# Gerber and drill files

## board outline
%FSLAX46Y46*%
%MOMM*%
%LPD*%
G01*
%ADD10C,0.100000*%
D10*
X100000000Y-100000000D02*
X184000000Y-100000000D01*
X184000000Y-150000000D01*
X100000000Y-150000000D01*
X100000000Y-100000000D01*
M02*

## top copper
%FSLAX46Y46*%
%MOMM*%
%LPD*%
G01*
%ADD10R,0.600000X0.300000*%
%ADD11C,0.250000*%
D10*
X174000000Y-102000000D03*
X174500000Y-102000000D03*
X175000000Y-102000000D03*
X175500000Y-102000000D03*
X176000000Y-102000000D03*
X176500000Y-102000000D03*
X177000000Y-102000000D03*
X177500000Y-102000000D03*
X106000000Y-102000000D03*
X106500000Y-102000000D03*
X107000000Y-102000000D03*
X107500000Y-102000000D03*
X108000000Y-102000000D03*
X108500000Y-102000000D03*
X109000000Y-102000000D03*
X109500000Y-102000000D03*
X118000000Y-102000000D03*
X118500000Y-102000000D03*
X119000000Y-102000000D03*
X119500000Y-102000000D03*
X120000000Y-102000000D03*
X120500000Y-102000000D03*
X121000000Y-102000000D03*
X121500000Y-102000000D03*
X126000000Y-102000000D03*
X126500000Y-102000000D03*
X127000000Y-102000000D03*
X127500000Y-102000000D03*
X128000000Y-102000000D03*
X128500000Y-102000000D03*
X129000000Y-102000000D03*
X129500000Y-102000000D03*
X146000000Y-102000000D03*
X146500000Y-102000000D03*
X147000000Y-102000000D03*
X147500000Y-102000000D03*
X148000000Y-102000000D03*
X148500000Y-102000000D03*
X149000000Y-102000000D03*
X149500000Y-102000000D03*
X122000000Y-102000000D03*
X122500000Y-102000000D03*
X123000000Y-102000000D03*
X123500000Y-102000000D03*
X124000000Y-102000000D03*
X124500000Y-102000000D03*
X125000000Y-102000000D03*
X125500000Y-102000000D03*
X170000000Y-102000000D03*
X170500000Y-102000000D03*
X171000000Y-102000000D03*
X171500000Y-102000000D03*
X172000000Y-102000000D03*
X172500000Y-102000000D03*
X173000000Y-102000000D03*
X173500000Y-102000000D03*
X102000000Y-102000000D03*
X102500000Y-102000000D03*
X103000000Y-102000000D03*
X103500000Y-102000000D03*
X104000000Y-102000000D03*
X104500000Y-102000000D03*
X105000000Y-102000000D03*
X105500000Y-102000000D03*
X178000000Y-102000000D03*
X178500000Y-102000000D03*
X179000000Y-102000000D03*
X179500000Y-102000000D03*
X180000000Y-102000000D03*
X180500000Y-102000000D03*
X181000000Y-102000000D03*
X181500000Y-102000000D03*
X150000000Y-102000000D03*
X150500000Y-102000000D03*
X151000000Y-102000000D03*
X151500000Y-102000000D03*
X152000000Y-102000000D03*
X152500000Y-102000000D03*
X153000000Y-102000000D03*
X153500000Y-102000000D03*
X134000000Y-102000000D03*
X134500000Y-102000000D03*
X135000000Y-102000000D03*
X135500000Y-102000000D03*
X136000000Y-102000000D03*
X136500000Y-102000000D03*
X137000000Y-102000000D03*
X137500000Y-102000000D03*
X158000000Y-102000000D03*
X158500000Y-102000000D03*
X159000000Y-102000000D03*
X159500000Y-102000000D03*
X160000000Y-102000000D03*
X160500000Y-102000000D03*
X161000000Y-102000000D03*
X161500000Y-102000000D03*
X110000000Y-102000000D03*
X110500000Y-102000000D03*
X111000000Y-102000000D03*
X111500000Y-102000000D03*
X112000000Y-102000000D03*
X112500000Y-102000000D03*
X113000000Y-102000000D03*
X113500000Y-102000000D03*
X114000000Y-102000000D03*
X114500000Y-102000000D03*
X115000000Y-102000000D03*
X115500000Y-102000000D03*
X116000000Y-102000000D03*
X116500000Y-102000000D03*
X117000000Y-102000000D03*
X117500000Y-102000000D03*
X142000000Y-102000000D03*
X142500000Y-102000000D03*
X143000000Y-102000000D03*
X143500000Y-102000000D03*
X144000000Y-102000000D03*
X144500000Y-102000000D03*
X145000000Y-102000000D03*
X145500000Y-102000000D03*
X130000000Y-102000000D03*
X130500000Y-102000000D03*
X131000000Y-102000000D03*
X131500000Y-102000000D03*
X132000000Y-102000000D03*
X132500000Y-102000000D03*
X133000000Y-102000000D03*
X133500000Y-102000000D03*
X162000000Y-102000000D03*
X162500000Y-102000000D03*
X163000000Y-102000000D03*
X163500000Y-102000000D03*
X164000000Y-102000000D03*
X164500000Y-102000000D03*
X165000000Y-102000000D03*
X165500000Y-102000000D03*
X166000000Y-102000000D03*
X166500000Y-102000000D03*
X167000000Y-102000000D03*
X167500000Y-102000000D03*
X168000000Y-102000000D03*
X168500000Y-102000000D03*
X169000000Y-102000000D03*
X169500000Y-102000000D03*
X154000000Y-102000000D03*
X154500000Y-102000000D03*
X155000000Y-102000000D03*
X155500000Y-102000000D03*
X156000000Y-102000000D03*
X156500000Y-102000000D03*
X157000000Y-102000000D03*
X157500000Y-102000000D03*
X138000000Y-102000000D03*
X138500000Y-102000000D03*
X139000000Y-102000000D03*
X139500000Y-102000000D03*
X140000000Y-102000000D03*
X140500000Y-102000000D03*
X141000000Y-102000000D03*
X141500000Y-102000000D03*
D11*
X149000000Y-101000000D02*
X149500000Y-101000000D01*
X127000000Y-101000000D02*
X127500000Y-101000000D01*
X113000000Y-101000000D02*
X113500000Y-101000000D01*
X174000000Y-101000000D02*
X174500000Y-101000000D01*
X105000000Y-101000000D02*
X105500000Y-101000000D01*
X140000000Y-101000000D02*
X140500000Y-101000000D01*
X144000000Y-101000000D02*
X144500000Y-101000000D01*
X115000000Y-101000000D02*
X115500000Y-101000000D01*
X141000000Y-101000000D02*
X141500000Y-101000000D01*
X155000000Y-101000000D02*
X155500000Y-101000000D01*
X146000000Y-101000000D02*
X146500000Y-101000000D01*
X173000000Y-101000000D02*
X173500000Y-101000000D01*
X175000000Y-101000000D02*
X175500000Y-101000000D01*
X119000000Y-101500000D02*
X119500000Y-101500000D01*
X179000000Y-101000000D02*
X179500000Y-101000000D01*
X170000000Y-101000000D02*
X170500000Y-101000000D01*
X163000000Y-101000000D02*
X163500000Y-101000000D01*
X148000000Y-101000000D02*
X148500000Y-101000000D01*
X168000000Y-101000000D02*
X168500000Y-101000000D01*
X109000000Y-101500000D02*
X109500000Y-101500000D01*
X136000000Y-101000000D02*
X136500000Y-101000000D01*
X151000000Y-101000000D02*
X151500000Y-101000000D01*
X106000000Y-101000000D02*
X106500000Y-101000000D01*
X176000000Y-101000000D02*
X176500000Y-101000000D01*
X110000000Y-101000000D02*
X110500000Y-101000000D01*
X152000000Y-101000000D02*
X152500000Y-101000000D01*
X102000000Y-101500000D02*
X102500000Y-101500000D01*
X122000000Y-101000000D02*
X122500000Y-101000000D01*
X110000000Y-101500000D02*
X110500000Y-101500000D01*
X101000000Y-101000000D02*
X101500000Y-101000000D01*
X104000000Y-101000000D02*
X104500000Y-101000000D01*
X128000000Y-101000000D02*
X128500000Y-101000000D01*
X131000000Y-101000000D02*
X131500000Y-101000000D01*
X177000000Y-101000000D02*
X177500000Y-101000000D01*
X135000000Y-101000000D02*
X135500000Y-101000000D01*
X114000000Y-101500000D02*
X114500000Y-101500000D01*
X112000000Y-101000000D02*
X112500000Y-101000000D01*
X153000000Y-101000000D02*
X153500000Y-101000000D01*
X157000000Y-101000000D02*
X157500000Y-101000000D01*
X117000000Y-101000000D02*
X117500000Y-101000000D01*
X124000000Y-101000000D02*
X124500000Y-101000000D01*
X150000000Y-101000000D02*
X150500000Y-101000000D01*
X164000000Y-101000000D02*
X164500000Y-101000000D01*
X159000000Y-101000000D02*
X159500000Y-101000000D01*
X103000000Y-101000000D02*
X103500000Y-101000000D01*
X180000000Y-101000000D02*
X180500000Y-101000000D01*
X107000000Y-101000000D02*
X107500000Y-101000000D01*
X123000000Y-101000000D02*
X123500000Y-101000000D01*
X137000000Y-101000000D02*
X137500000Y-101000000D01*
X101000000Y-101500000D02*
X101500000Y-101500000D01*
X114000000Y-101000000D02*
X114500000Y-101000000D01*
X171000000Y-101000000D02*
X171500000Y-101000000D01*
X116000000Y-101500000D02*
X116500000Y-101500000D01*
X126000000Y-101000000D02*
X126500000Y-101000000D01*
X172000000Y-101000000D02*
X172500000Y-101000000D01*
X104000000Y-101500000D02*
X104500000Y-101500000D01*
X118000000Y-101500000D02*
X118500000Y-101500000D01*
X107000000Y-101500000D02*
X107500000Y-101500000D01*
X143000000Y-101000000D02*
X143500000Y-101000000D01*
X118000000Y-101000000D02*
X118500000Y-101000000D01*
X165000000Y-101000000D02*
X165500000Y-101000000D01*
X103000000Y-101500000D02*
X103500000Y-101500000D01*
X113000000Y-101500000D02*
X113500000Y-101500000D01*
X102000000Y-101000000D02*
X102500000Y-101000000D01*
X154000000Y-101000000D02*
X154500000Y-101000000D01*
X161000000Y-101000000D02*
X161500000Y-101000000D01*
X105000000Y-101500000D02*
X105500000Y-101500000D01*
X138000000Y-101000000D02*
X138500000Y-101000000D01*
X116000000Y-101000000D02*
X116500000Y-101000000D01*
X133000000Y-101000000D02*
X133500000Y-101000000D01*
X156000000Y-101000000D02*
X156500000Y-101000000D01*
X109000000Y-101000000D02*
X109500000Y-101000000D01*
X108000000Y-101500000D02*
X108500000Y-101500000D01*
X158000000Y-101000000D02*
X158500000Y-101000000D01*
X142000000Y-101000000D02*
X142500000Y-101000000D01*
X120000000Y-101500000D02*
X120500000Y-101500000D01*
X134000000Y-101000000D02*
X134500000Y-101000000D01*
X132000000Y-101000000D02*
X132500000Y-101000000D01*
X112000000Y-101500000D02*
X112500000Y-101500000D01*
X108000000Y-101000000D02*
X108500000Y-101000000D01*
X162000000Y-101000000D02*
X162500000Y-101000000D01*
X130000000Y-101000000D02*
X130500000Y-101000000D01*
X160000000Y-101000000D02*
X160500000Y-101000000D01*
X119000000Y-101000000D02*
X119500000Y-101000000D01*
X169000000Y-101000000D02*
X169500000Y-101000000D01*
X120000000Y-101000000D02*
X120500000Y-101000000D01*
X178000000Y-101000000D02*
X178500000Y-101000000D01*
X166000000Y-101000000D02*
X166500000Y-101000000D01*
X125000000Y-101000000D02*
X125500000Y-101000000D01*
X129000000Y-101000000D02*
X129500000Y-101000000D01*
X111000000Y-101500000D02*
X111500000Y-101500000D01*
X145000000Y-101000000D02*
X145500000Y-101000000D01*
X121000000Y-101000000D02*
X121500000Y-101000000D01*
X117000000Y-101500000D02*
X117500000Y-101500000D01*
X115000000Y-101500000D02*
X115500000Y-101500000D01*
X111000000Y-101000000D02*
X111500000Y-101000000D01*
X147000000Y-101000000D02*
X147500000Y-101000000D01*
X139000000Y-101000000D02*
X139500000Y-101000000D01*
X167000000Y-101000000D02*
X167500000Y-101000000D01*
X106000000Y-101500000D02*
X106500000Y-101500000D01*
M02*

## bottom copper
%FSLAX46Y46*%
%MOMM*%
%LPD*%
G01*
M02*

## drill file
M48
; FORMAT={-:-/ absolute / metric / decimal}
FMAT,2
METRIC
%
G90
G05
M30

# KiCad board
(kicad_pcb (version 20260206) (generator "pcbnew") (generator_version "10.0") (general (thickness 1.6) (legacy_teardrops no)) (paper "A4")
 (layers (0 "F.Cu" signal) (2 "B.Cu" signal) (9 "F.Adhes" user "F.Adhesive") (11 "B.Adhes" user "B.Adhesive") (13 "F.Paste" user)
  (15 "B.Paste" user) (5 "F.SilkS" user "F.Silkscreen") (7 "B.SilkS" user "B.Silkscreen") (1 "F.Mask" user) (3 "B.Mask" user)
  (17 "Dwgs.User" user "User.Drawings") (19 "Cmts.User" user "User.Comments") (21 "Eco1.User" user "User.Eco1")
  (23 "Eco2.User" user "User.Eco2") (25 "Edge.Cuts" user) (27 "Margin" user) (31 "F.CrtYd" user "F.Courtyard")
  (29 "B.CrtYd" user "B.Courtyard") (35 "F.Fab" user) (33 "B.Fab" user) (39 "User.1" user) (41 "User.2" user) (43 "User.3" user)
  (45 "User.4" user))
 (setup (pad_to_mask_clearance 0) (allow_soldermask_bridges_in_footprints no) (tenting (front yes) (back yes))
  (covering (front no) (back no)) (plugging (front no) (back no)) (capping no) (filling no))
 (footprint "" (layer "F.Cu") (at 174 102)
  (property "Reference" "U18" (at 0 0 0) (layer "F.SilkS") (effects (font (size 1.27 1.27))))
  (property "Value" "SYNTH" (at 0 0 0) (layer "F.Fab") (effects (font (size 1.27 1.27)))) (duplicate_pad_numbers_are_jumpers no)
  (pad "1" smd rect (at 0 0) (size 0.6 0.3) (layers "F.Cu" "F.Mask" "F.Paste") (thermal_bridge_angle 45))
  (pad "2" smd rect (at 0.5 0) (size 0.6 0.3) (layers "F.Cu" "F.Mask" "F.Paste") (thermal_bridge_angle 45))
  (pad "3" smd rect (at 1 0) (size 0.6 0.3) (layers "F.Cu" "F.Mask" "F.Paste") (thermal_bridge_angle 45))
  (pad "4" smd rect (at 1.5 0) (size 0.6 0.3) (layers "F.Cu" "F.Mask" "F.Paste") (thermal_bridge_angle 45))
  (pad "5" smd rect (at 2 0) (size 0.6 0.3) (layers "F.Cu" "F.Mask" "F.Paste") (thermal_bridge_angle 45))
  (pad "6" smd rect (at 2.5 0) (size 0.6 0.3) (layers "F.Cu" "F.Mask" "F.Paste") (thermal_bridge_angle 45))
  (pad "7" smd rect (at 3 0) (size 0.6 0.3) (layers "F.Cu" "F.Mask" "F.Paste") (thermal_bridge_angle 45))
  (pad "8" smd rect (at 3.5 0) (size 0.6 0.3) (layers "F.Cu" "F.Mask" "F.Paste") (thermal_bridge_angle 45)))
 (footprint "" (layer "F.Cu") (at 106 102)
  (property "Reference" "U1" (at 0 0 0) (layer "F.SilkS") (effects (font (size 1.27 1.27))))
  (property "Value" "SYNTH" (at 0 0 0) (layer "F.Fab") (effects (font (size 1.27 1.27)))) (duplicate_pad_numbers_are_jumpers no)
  (pad "1" smd rect (at 0 0) (size 0.6 0.3) (layers "F.Cu" "F.Mask" "F.Paste") (thermal_bridge_angle 45))
  (pad "2" smd rect (at 0.5 0) (size 0.6 0.3) (layers "F.Cu" "F.Mask" "F.Paste") (thermal_bridge_angle 45))
  (pad "3" smd rect (at 1 0) (size 0.6 0.3) (layers "F.Cu" "F.Mask" "F.Paste") (thermal_bridge_angle 45))
  (pad "4" smd rect (at 1.5 0) (size 0.6 0.3) (layers "F.Cu" "F.Mask" "F.Paste") (thermal_bridge_angle 45))
  (pad "5" smd rect (at 2 0) (size 0.6 0.3) (layers "F.Cu" "F.Mask" "F.Paste") (thermal_bridge_angle 45))
  (pad "6" smd rect (at 2.5 0) (size 0.6 0.3) (layers "F.Cu" "F.Mask" "F.Paste") (thermal_bridge_angle 45))
  (pad "7" smd rect (at 3 0) (size 0.6 0.3) (layers "F.Cu" "F.Mask" "F.Paste") (thermal_bridge_angle 45))
  (pad "8" smd rect (at 3.5 0) (size 0.6 0.3) (layers "F.Cu" "F.Mask" "F.Paste") (thermal_bridge_angle 45)))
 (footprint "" (layer "F.Cu") (at 118 102)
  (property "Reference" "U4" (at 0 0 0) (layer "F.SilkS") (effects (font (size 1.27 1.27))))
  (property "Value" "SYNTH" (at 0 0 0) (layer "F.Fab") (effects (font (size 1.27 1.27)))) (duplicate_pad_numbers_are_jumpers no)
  (pad "1" smd rect (at 0 0) (size 0.6 0.3) (layers "F.Cu" "F.Mask" "F.Paste") (thermal_bridge_angle 45))
  (pad "2" smd rect (at 0.5 0) (size 0.6 0.3) (layers "F.Cu" "F.Mask" "F.Paste") (thermal_bridge_angle 45))
  (pad "3" smd rect (at 1 0) (size 0.6 0.3) (layers "F.Cu" "F.Mask" "F.Paste") (thermal_bridge_angle 45))
  (pad "4" smd rect (at 1.5 0) (size 0.6 0.3) (layers "F.Cu" "F.Mask" "F.Paste") (thermal_bridge_angle 45))
  (pad "5" smd rect (at 2 0) (size 0.6 0.3) (layers "F.Cu" "F.Mask" "F.Paste") (thermal_bridge_angle 45))
  (pad "6" smd rect (at 2.5 0) (size 0.6 0.3) (layers "F.Cu" "F.Mask" "F.Paste") (thermal_bridge_angle 45))
  (pad "7" smd rect (at 3 0) (size 0.6 0.3) (layers "F.Cu" "F.Mask" "F.Paste") (thermal_bridge_angle 45))
  (pad "8" smd rect (at 3.5 0) (size 0.6 0.3) (layers "F.Cu" "F.Mask" "F.Paste") (thermal_bridge_angle 45)))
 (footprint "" (layer "F.Cu") (at 126 102)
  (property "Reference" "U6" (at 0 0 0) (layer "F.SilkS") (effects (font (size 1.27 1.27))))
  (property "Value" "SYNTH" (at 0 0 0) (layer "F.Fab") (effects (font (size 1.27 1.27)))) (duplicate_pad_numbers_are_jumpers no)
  (pad "1" smd rect (at 0 0) (size 0.6 0.3) (layers "F.Cu" "F.Mask" "F.Paste") (thermal_bridge_angle 45))
  (pad "2" smd rect (at 0.5 0) (size 0.6 0.3) (layers "F.Cu" "F.Mask" "F.Paste") (thermal_bridge_angle 45))
  (pad "3" smd rect (at 1 0) (size 0.6 0.3) (layers "F.Cu" "F.Mask" "F.Paste") (thermal_bridge_angle 45))
  (pad "4" smd rect (at 1.5 0) (size 0.6 0.3) (layers "F.Cu" "F.Mask" "F.Paste") (thermal_bridge_angle 45))
  (pad "5" smd rect (at 2 0) (size 0.6 0.3) (layers "F.Cu" "F.Mask" "F.Paste") (thermal_bridge_angle 45))
  (pad "6" smd rect (at 2.5 0) (size 0.6 0.3) (layers "F.Cu" "F.Mask" "F.Paste") (thermal_bridge_angle 45))
  (pad "7" smd rect (at 3 0) (size 0.6 0.3) (layers "F.Cu" "F.Mask" "F.Paste") (thermal_bridge_angle 45))
  (pad "8" smd rect (at 3.5 0) (size 0.6 0.3) (layers "F.Cu" "F.Mask" "F.Paste") (thermal_bridge_angle 45)))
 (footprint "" (layer "F.Cu") (at 146 102)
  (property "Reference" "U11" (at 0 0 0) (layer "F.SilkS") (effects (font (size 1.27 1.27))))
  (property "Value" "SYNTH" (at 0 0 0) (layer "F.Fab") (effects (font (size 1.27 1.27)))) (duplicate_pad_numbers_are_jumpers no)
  (pad "1" smd rect (at 0 0) (size 0.6 0.3) (layers "F.Cu" "F.Mask" "F.Paste") (thermal_bridge_angle 45))
  (pad "2" smd rect (at 0.5 0) (size 0.6 0.3) (layers "F.Cu" "F.Mask" "F.Paste") (thermal_bridge_angle 45))
  (pad "3" smd rect (at 1 0) (size 0.6 0.3) (layers "F.Cu" "F.Mask" "F.Paste") (thermal_bridge_angle 45))
  (pad "4" smd rect (at 1.5 0) (size 0.6 0.3) (layers "F.Cu" "F.Mask" "F.Paste") (thermal_bridge_angle 45))
  (pad "5" smd rect (at 2 0) (size 0.6 0.3) (layers "F.Cu" "F.Mask" "F.Paste") (thermal_bridge_angle 45))
  (pad "6" smd rect (at 2.5 0) (size 0.6 0.3) (layers "F.Cu" "F.Mask" "F.Paste") (thermal_bridge_angle 45))
  (pad "7" smd rect (at 3 0) (size 0.6 0.3) (layers "F.Cu" "F.Mask" "F.Paste") (thermal_bridge_angle 45))
  (pad "8" smd rect (at 3.5 0) (size 0.6 0.3) (layers "F.Cu" "F.Mask" "F.Paste") (thermal_bridge_angle 45)))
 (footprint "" (layer "F.Cu") (at 122 102)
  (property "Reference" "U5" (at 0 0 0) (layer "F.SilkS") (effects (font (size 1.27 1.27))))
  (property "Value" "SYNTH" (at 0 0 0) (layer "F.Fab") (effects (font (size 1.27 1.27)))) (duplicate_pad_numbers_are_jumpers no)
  (pad "1" smd rect (at 0 0) (size 0.6 0.3) (layers "F.Cu" "F.Mask" "F.Paste") (thermal_bridge_angle 45))
  (pad "2" smd rect (at 0.5 0) (size 0.6 0.3) (layers "F.Cu" "F.Mask" "F.Paste") (thermal_bridge_angle 45))
  (pad "3" smd rect (at 1 0) (size 0.6 0.3) (layers "F.Cu" "F.Mask" "F.Paste") (thermal_bridge_angle 45))
  (pad "4" smd rect (at 1.5 0) (size 0.6 0.3) (layers "F.Cu" "F.Mask" "F.Paste") (thermal_bridge_angle 45))
  (pad "5" smd rect (at 2 0) (size 0.6 0.3) (layers "F.Cu" "F.Mask" "F.Paste") (thermal_bridge_angle 45))
  (pad "6" smd rect (at 2.5 0) (size 0.6 0.3) (layers "F.Cu" "F.Mask" "F.Paste") (thermal_bridge_angle 45))
  (pad "7" smd rect (at 3 0) (size 0.6 0.3) (layers "F.Cu" "F.Mask" "F.Paste") (thermal_bridge_angle 45))
  (pad "8" smd rect (at 3.5 0) (size 0.6 0.3) (layers "F.Cu" "F.Mask" "F.Paste") (thermal_bridge_angle 45)))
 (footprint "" (layer "F.Cu") (at 170 102)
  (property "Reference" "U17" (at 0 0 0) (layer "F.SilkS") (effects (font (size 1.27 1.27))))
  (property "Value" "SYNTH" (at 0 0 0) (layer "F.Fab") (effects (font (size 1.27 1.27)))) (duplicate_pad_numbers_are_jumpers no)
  (pad "1" smd rect (at 0 0) (size 0.6 0.3) (layers "F.Cu" "F.Mask" "F.Paste") (thermal_bridge_angle 45))
  (pad "2" smd rect (at 0.5 0) (size 0.6 0.3) (layers "F.Cu" "F.Mask" "F.Paste") (thermal_bridge_angle 45))
  (pad "3" smd rect (at 1 0) (size 0.6 0.3) (layers "F.Cu" "F.Mask" "F.Paste") (thermal_bridge_angle 45))
  (pad "4" smd rect (at 1.5 0) (size 0.6 0.3) (layers "F.Cu" "F.Mask" "F.Paste") (thermal_bridge_angle 45))
  (pad "5" smd rect (at 2 0) (size 0.6 0.3) (layers "F.Cu" "F.Mask" "F.Paste") (thermal_bridge_angle 45))
  (pad "6" smd rect (at 2.5 0) (size 0.6 0.3) (layers "F.Cu" "F.Mask" "F.Paste") (thermal_bridge_angle 45))
  (pad "7" smd rect (at 3 0) (size 0.6 0.3) (layers "F.Cu" "F.Mask" "F.Paste") (thermal_bridge_angle 45))
  (pad "8" smd rect (at 3.5 0) (size 0.6 0.3) (layers "F.Cu" "F.Mask" "F.Paste") (thermal_bridge_angle 45)))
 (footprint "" (layer "F.Cu") (at 102 102)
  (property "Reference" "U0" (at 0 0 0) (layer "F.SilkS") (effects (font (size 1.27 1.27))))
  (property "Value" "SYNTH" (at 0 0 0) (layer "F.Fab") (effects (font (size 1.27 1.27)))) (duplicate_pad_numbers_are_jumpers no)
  (pad "1" smd rect (at 0 0) (size 0.6 0.3) (layers "F.Cu" "F.Mask" "F.Paste") (thermal_bridge_angle 45))
  (pad "2" smd rect (at 0.5 0) (size 0.6 0.3) (layers "F.Cu" "F.Mask" "F.Paste") (thermal_bridge_angle 45))
  (pad "3" smd rect (at 1 0) (size 0.6 0.3) (layers "F.Cu" "F.Mask" "F.Paste") (thermal_bridge_angle 45))
  (pad "4" smd rect (at 1.5 0) (size 0.6 0.3) (layers "F.Cu" "F.Mask" "F.Paste") (thermal_bridge_angle 45))
  (pad "5" smd rect (at 2 0) (size 0.6 0.3) (layers "F.Cu" "F.Mask" "F.Paste") (thermal_bridge_angle 45))
  (pad "6" smd rect (at 2.5 0) (size 0.6 0.3) (layers "F.Cu" "F.Mask" "F.Paste") (thermal_bridge_angle 45))
  (pad "7" smd rect (at 3 0) (size 0.6 0.3) (layers "F.Cu" "F.Mask" "F.Paste") (thermal_bridge_angle 45))
  (pad "8" smd rect (at 3.5 0) (size 0.6 0.3) (layers "F.Cu" "F.Mask" "F.Paste") (thermal_bridge_angle 45)))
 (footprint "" (layer "F.Cu") (at 178 102)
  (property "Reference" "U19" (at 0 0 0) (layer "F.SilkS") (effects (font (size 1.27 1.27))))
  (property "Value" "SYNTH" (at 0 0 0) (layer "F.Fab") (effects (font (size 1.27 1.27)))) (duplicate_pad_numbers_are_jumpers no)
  (pad "1" smd rect (at 0 0) (size 0.6 0.3) (layers "F.Cu" "F.Mask" "F.Paste") (thermal_bridge_angle 45))
  (pad "2" smd rect (at 0.5 0) (size 0.6 0.3) (layers "F.Cu" "F.Mask" "F.Paste") (thermal_bridge_angle 45))
  (pad "3" smd rect (at 1 0) (size 0.6 0.3) (layers "F.Cu" "F.Mask" "F.Paste") (thermal_bridge_angle 45))
  (pad "4" smd rect (at 1.5 0) (size 0.6 0.3) (layers "F.Cu" "F.Mask" "F.Paste") (thermal_bridge_angle 45))
  (pad "5" smd rect (at 2 0) (size 0.6 0.3) (layers "F.Cu" "F.Mask" "F.Paste") (thermal_bridge_angle 45))
  (pad "6" smd rect (at 2.5 0) (size 0.6 0.3) (layers "F.Cu" "F.Mask" "F.Paste") (thermal_bridge_angle 45))
  (pad "7" smd rect (at 3 0) (size 0.6 0.3) (layers "F.Cu" "F.Mask" "F.Paste") (thermal_bridge_angle 45))
  (pad "8" smd rect (at 3.5 0) (size 0.6 0.3) (layers "F.Cu" "F.Mask" "F.Paste") (thermal_bridge_angle 45)))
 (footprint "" (layer "F.Cu") (at 150 102)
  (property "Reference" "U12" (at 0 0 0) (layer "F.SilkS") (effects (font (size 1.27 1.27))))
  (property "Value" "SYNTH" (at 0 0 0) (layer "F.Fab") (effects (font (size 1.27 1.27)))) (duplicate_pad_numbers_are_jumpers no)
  (pad "1" smd rect (at 0 0) (size 0.6 0.3) (layers "F.Cu" "F.Mask" "F.Paste") (thermal_bridge_angle 45))
  (pad "2" smd rect (at 0.5 0) (size 0.6 0.3) (layers "F.Cu" "F.Mask" "F.Paste") (thermal_bridge_angle 45))
  (pad "3" smd rect (at 1 0) (size 0.6 0.3) (layers "F.Cu" "F.Mask" "F.Paste") (thermal_bridge_angle 45))
  (pad "4" smd rect (at 1.5 0) (size 0.6 0.3) (layers "F.Cu" "F.Mask" "F.Paste") (thermal_bridge_angle 45))
  (pad "5" smd rect (at 2 0) (size 0.6 0.3) (layers "F.Cu" "F.Mask" "F.Paste") (thermal_bridge_angle 45))
  (pad "6" smd rect (at 2.5 0) (size 0.6 0.3) (layers "F.Cu" "F.Mask" "F.Paste") (thermal_bridge_angle 45))
  (pad "7" smd rect (at 3 0) (size 0.6 0.3) (layers "F.Cu" "F.Mask" "F.Paste") (thermal_bridge_angle 45))
  (pad "8" smd rect (at 3.5 0) (size 0.6 0.3) (layers "F.Cu" "F.Mask" "F.Paste") (thermal_bridge_angle 45)))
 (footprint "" (layer "F.Cu") (at 134 102)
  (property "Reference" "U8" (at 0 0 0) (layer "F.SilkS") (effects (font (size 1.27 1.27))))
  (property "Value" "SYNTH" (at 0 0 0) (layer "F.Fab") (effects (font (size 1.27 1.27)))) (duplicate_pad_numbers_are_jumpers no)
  (pad "1" smd rect (at 0 0) (size 0.6 0.3) (layers "F.Cu" "F.Mask" "F.Paste") (thermal_bridge_angle 45))
  (pad "2" smd rect (at 0.5 0) (size 0.6 0.3) (layers "F.Cu" "F.Mask" "F.Paste") (thermal_bridge_angle 45))
  (pad "3" smd rect (at 1 0) (size 0.6 0.3) (layers "F.Cu" "F.Mask" "F.Paste") (thermal_bridge_angle 45))
  (pad "4" smd rect (at 1.5 0) (size 0.6 0.3) (layers "F.Cu" "F.Mask" "F.Paste") (thermal_bridge_angle 45))
  (pad "5" smd rect (at 2 0) (size 0.6 0.3) (layers "F.Cu" "F.Mask" "F.Paste") (thermal_bridge_angle 45))
  (pad "6" smd rect (at 2.5 0) (size 0.6 0.3) (layers "F.Cu" "F.Mask" "F.Paste") (thermal_bridge_angle 45))
  (pad "7" smd rect (at 3 0) (size 0.6 0.3) (layers "F.Cu" "F.Mask" "F.Paste") (thermal_bridge_angle 45))
  (pad "8" smd rect (at 3.5 0) (size 0.6 0.3) (layers "F.Cu" "F.Mask" "F.Paste") (thermal_bridge_angle 45)))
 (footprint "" (layer "F.Cu") (at 158 102)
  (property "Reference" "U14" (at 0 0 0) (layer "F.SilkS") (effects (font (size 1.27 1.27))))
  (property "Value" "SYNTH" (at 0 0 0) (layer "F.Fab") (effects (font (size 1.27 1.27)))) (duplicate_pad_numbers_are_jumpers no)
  (pad "1" smd rect (at 0 0) (size 0.6 0.3) (layers "F.Cu" "F.Mask" "F.Paste") (thermal_bridge_angle 45))
  (pad "2" smd rect (at 0.5 0) (size 0.6 0.3) (layers "F.Cu" "F.Mask" "F.Paste") (thermal_bridge_angle 45))
  (pad "3" smd rect (at 1 0) (size 0.6 0.3) (layers "F.Cu" "F.Mask" "F.Paste") (thermal_bridge_angle 45))
  (pad "4" smd rect (at 1.5 0) (size 0.6 0.3) (layers "F.Cu" "F.Mask" "F.Paste") (thermal_bridge_angle 45))
  (pad "5" smd rect (at 2 0) (size 0.6 0.3) (layers "F.Cu" "F.Mask" "F.Paste") (thermal_bridge_angle 45))
  (pad "6" smd rect (at 2.5 0) (size 0.6 0.3) (layers "F.Cu" "F.Mask" "F.Paste") (thermal_bridge_angle 45))
  (pad "7" smd rect (at 3 0) (size 0.6 0.3) (layers "F.Cu" "F.Mask" "F.Paste") (thermal_bridge_angle 45))
  (pad "8" smd rect (at 3.5 0) (size 0.6 0.3) (layers "F.Cu" "F.Mask" "F.Paste") (thermal_bridge_angle 45)))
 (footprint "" (layer "F.Cu") (at 110 102)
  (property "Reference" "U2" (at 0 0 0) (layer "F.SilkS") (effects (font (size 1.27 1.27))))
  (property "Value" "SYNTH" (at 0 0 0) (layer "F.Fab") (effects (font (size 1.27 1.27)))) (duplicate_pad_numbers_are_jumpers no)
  (pad "1" smd rect (at 0 0) (size 0.6 0.3) (layers "F.Cu" "F.Mask" "F.Paste") (thermal_bridge_angle 45))
  (pad "2" smd rect (at 0.5 0) (size 0.6 0.3) (layers "F.Cu" "F.Mask" "F.Paste") (thermal_bridge_angle 45))
  (pad "3" smd rect (at 1 0) (size 0.6 0.3) (layers "F.Cu" "F.Mask" "F.Paste") (thermal_bridge_angle 45))
  (pad "4" smd rect (at 1.5 0) (size 0.6 0.3) (layers "F.Cu" "F.Mask" "F.Paste") (thermal_bridge_angle 45))
  (pad "5" smd rect (at 2 0) (size 0.6 0.3) (layers "F.Cu" "F.Mask" "F.Paste") (thermal_bridge_angle 45))
  (pad "6" smd rect (at 2.5 0) (size 0.6 0.3) (layers "F.Cu" "F.Mask" "F.Paste") (thermal_bridge_angle 45))
  (pad "7" smd rect (at 3 0) (size 0.6 0.3) (layers "F.Cu" "F.Mask" "F.Paste") (thermal_bridge_angle 45))
  (pad "8" smd rect (at 3.5 0) (size 0.6 0.3) (layers "F.Cu" "F.Mask" "F.Paste") (thermal_bridge_angle 45)))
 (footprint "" (layer "F.Cu") (at 114 102)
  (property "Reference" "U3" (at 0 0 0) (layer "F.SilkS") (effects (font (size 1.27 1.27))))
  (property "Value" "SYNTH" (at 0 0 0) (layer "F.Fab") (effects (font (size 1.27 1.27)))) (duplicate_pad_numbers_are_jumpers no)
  (pad "1" smd rect (at 0 0) (size 0.6 0.3) (layers "F.Cu" "F.Mask" "F.Paste") (thermal_bridge_angle 45))
  (pad "2" smd rect (at 0.5 0) (size 0.6 0.3) (layers "F.Cu" "F.Mask" "F.Paste") (thermal_bridge_angle 45))
  (pad "3" smd rect (at 1 0) (size 0.6 0.3) (layers "F.Cu" "F.Mask" "F.Paste") (thermal_bridge_angle 45))
  (pad "4" smd rect (at 1.5 0) (size 0.6 0.3) (layers "F.Cu" "F.Mask" "F.Paste") (thermal_bridge_angle 45))
  (pad "5" smd rect (at 2 0) (size 0.6 0.3) (layers "F.Cu" "F.Mask" "F.Paste") (thermal_bridge_angle 45))
  (pad "6" smd rect (at 2.5 0) (size 0.6 0.3) (layers "F.Cu" "F.Mask" "F.Paste") (thermal_bridge_angle 45))
  (pad "7" smd rect (at 3 0) (size 0.6 0.3) (layers "F.Cu" "F.Mask" "F.Paste") (thermal_bridge_angle 45))
  (pad "8" smd rect (at 3.5 0) (size 0.6 0.3) (layers "F.Cu" "F.Mask" "F.Paste") (thermal_bridge_angle 45)))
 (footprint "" (layer "F.Cu") (at 142 102)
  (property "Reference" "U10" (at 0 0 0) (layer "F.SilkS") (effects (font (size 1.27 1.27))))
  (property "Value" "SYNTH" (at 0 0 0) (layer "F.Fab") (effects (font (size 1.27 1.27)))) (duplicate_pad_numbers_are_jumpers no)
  (pad "1" smd rect (at 0 0) (size 0.6 0.3) (layers "F.Cu" "F.Mask" "F.Paste") (thermal_bridge_angle 45))
  (pad "2" smd rect (at 0.5 0) (size 0.6 0.3) (layers "F.Cu" "F.Mask" "F.Paste") (thermal_bridge_angle 45))
  (pad "3" smd rect (at 1 0) (size 0.6 0.3) (layers "F.Cu" "F.Mask" "F.Paste") (thermal_bridge_angle 45))
  (pad "4" smd rect (at 1.5 0) (size 0.6 0.3) (layers "F.Cu" "F.Mask" "F.Paste") (thermal_bridge_angle 45))
  (pad "5" smd rect (at 2 0) (size 0.6 0.3) (layers "F.Cu" "F.Mask" "F.Paste") (thermal_bridge_angle 45))
  (pad "6" smd rect (at 2.5 0) (size 0.6 0.3) (layers "F.Cu" "F.Mask" "F.Paste") (thermal_bridge_angle 45))
  (pad "7" smd rect (at 3 0) (size 0.6 0.3) (layers "F.Cu" "F.Mask" "F.Paste") (thermal_bridge_angle 45))
  (pad "8" smd rect (at 3.5 0) (size 0.6 0.3) (layers "F.Cu" "F.Mask" "F.Paste") (thermal_bridge_angle 45)))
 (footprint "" (layer "F.Cu") (at 130 102)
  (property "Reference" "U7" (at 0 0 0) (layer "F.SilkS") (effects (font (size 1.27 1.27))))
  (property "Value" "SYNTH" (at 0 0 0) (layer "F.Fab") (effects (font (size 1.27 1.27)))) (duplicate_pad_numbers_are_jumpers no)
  (pad "1" smd rect (at 0 0) (size 0.6 0.3) (layers "F.Cu" "F.Mask" "F.Paste") (thermal_bridge_angle 45))
  (pad "2" smd rect (at 0.5 0) (size 0.6 0.3) (layers "F.Cu" "F.Mask" "F.Paste") (thermal_bridge_angle 45))
  (pad "3" smd rect (at 1 0) (size 0.6 0.3) (layers "F.Cu" "F.Mask" "F.Paste") (thermal_bridge_angle 45))
  (pad "4" smd rect (at 1.5 0) (size 0.6 0.3) (layers "F.Cu" "F.Mask" "F.Paste") (thermal_bridge_angle 45))
  (pad "5" smd rect (at 2 0) (size 0.6 0.3) (layers "F.Cu" "F.Mask" "F.Paste") (thermal_bridge_angle 45))
  (pad "6" smd rect (at 2.5 0) (size 0.6 0.3) (layers "F.Cu" "F.Mask" "F.Paste") (thermal_bridge_angle 45))
  (pad "7" smd rect (at 3 0) (size 0.6 0.3) (layers "F.Cu" "F.Mask" "F.Paste") (thermal_bridge_angle 45))
  (pad "8" smd rect (at 3.5 0) (size 0.6 0.3) (layers "F.Cu" "F.Mask" "F.Paste") (thermal_bridge_angle 45)))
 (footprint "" (layer "F.Cu") (at 162 102)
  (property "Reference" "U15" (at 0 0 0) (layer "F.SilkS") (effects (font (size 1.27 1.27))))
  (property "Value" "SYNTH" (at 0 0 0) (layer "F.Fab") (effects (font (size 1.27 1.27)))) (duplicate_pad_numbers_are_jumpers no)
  (pad "1" smd rect (at 0 0) (size 0.6 0.3) (layers "F.Cu" "F.Mask" "F.Paste") (thermal_bridge_angle 45))
  (pad "2" smd rect (at 0.5 0) (size 0.6 0.3) (layers "F.Cu" "F.Mask" "F.Paste") (thermal_bridge_angle 45))
  (pad "3" smd rect (at 1 0) (size 0.6 0.3) (layers "F.Cu" "F.Mask" "F.Paste") (thermal_bridge_angle 45))
  (pad "4" smd rect (at 1.5 0) (size 0.6 0.3) (layers "F.Cu" "F.Mask" "F.Paste") (thermal_bridge_angle 45))
  (pad "5" smd rect (at 2 0) (size 0.6 0.3) (layers "F.Cu" "F.Mask" "F.Paste") (thermal_bridge_angle 45))
  (pad "6" smd rect (at 2.5 0) (size 0.6 0.3) (layers "F.Cu" "F.Mask" "F.Paste") (thermal_bridge_angle 45))
  (pad "7" smd rect (at 3 0) (size 0.6 0.3) (layers "F.Cu" "F.Mask" "F.Paste") (thermal_bridge_angle 45))
  (pad "8" smd rect (at 3.5 0) (size 0.6 0.3) (layers "F.Cu" "F.Mask" "F.Paste") (thermal_bridge_angle 45)))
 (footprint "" (layer "F.Cu") (at 166 102)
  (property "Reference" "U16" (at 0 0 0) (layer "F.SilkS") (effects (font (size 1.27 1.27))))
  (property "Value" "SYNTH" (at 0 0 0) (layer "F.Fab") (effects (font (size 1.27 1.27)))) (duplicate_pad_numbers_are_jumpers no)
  (pad "1" smd rect (at 0 0) (size 0.6 0.3) (layers "F.Cu" "F.Mask" "F.Paste") (thermal_bridge_angle 45))
  (pad "2" smd rect (at 0.5 0) (size 0.6 0.3) (layers "F.Cu" "F.Mask" "F.Paste") (thermal_bridge_angle 45))
  (pad "3" smd rect (at 1 0) (size 0.6 0.3) (layers "F.Cu" "F.Mask" "F.Paste") (thermal_bridge_angle 45))
  (pad "4" smd rect (at 1.5 0) (size 0.6 0.3) (layers "F.Cu" "F.Mask" "F.Paste") (thermal_bridge_angle 45))
  (pad "5" smd rect (at 2 0) (size 0.6 0.3) (layers "F.Cu" "F.Mask" "F.Paste") (thermal_bridge_angle 45))
  (pad "6" smd rect (at 2.5 0) (size 0.6 0.3) (layers "F.Cu" "F.Mask" "F.Paste") (thermal_bridge_angle 45))
  (pad "7" smd rect (at 3 0) (size 0.6 0.3) (layers "F.Cu" "F.Mask" "F.Paste") (thermal_bridge_angle 45))
  (pad "8" smd rect (at 3.5 0) (size 0.6 0.3) (layers "F.Cu" "F.Mask" "F.Paste") (thermal_bridge_angle 45)))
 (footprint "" (layer "F.Cu") (at 154 102)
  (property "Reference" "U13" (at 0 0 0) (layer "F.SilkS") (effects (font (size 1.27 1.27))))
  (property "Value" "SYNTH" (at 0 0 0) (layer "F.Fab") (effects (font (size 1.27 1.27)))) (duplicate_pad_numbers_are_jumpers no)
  (pad "1" smd rect (at 0 0) (size 0.6 0.3) (layers "F.Cu" "F.Mask" "F.Paste") (thermal_bridge_angle 45))
  (pad "2" smd rect (at 0.5 0) (size 0.6 0.3) (layers "F.Cu" "F.Mask" "F.Paste") (thermal_bridge_angle 45))
  (pad "3" smd rect (at 1 0) (size 0.6 0.3) (layers "F.Cu" "F.Mask" "F.Paste") (thermal_bridge_angle 45))
  (pad "4" smd rect (at 1.5 0) (size 0.6 0.3) (layers "F.Cu" "F.Mask" "F.Paste") (thermal_bridge_angle 45))
  (pad "5" smd rect (at 2 0) (size 0.6 0.3) (layers "F.Cu" "F.Mask" "F.Paste") (thermal_bridge_angle 45))
  (pad "6" smd rect (at 2.5 0) (size 0.6 0.3) (layers "F.Cu" "F.Mask" "F.Paste") (thermal_bridge_angle 45))
  (pad "7" smd rect (at 3 0) (size 0.6 0.3) (layers "F.Cu" "F.Mask" "F.Paste") (thermal_bridge_angle 45))
  (pad "8" smd rect (at 3.5 0) (size 0.6 0.3) (layers "F.Cu" "F.Mask" "F.Paste") (thermal_bridge_angle 45)))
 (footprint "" (layer "F.Cu") (at 138 102)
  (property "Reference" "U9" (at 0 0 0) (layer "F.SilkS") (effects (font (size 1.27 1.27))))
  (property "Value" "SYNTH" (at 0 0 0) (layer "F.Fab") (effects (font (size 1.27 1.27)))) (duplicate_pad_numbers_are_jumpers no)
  (pad "1" smd rect (at 0 0) (size 0.6 0.3) (layers "F.Cu" "F.Mask" "F.Paste") (thermal_bridge_angle 45))
  (pad "2" smd rect (at 0.5 0) (size 0.6 0.3) (layers "F.Cu" "F.Mask" "F.Paste") (thermal_bridge_angle 45))
  (pad "3" smd rect (at 1 0) (size 0.6 0.3) (layers "F.Cu" "F.Mask" "F.Paste") (thermal_bridge_angle 45))
  (pad "4" smd rect (at 1.5 0) (size 0.6 0.3) (layers "F.Cu" "F.Mask" "F.Paste") (thermal_bridge_angle 45))
  (pad "5" smd rect (at 2 0) (size 0.6 0.3) (layers "F.Cu" "F.Mask" "F.Paste") (thermal_bridge_angle 45))
  (pad "6" smd rect (at 2.5 0) (size 0.6 0.3) (layers "F.Cu" "F.Mask" "F.Paste") (thermal_bridge_angle 45))
  (pad "7" smd rect (at 3 0) (size 0.6 0.3) (layers "F.Cu" "F.Mask" "F.Paste") (thermal_bridge_angle 45))
  (pad "8" smd rect (at 3.5 0) (size 0.6 0.3) (layers "F.Cu" "F.Mask" "F.Paste") (thermal_bridge_angle 45)))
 (gr_rect (start 100 100) (end 184 150) (stroke (width 0.1) (type default)) (fill no) (layer "Edge.Cuts"))
 (segment (start 149 101) (end 149.5 101) (width 0.25) (layer "F.Cu") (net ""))
 (segment (start 127 101) (end 127.5 101) (width 0.25) (layer "F.Cu") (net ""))
 (segment (start 113 101) (end 113.5 101) (width 0.25) (layer "F.Cu") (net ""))
 (segment (start 174 101) (end 174.5 101) (width 0.25) (layer "F.Cu") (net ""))
 (segment (start 105 101) (end 105.5 101) (width 0.25) (layer "F.Cu") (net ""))
 (segment (start 140 101) (end 140.5 101) (width 0.25) (layer "F.Cu") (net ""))
 (segment (start 144 101) (end 144.5 101) (width 0.25) (layer "F.Cu") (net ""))
 (segment (start 115 101) (end 115.5 101) (width 0.25) (layer "F.Cu") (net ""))
 (segment (start 141 101) (end 141.5 101) (width 0.25) (layer "F.Cu") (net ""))
 (segment (start 155 101) (end 155.5 101) (width 0.25) (layer "F.Cu") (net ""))
 (segment (start 146 101) (end 146.5 101) (width 0.25) (layer "F.Cu") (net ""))
 (segment (start 173 101) (end 173.5 101) (width 0.25) (layer "F.Cu") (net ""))
 (segment (start 175 101) (end 175.5 101) (width 0.25) (layer "F.Cu") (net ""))
 (segment (start 119 101.5) (end 119.5 101.5) (width 0.25) (layer "F.Cu") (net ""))
 (segment (start 179 101) (end 179.5 101) (width 0.25) (layer "F.Cu") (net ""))
 (segment (start 170 101) (end 170.5 101) (width 0.25) (layer "F.Cu") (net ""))
 (segment (start 163 101) (end 163.5 101) (width 0.25) (layer "F.Cu") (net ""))
 (segment (start 148 101) (end 148.5 101) (width 0.25) (layer "F.Cu") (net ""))
 (segment (start 168 101) (end 168.5 101) (width 0.25) (layer "F.Cu") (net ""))
 (segment (start 109 101.5) (end 109.5 101.5) (width 0.25) (layer "F.Cu") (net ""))
 (segment (start 136 101) (end 136.5 101) (width 0.25) (layer "F.Cu") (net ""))
 (segment (start 151 101) (end 151.5 101) (width 0.25) (layer "F.Cu") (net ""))
 (segment (start 106 101) (end 106.5 101) (width 0.25) (layer "F.Cu") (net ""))
 (segment (start 176 101) (end 176.5 101) (width 0.25) (layer "F.Cu") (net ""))
 (segment (start 110 101) (end 110.5 101) (width 0.25) (layer "F.Cu") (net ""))
 (segment (start 152 101) (end 152.5 101) (width 0.25) (layer "F.Cu") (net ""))
 (segment (start 102 101.5) (end 102.5 101.5) (width 0.25) (layer "F.Cu") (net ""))
 (segment (start 122 101) (end 122.5 101) (width 0.25) (layer "F.Cu") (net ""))
 (segment (start 110 101.5) (end 110.5 101.5) (width 0.25) (layer "F.Cu") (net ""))
 (segment (start 101 101) (end 101.5 101) (width 0.25) (layer "F.Cu") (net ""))
 (segment (start 104 101) (end 104.5 101) (width 0.25) (layer "F.Cu") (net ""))
 (segment (start 128 101) (end 128.5 101) (width 0.25) (layer "F.Cu") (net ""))
 (segment (start 131 101) (end 131.5 101) (width 0.25) (layer "F.Cu") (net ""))
 (segment (start 177 101) (end 177.5 101) (width 0.25) (layer "F.Cu") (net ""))
 (segment (start 135 101) (end 135.5 101) (width 0.25) (layer "F.Cu") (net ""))
 (segment (start 114 101.5) (end 114.5 101.5) (width 0.25) (layer "F.Cu") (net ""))
 (segment (start 112 101) (end 112.5 101) (width 0.25) (layer "F.Cu") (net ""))
 (segment (start 153 101) (end 153.5 101) (width 0.25) (layer "F.Cu") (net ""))
 (segment (start 157 101) (end 157.5 101) (width 0.25) (layer "F.Cu") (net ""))
 (segment (start 117 101) (end 117.5 101) (width 0.25) (layer "F.Cu") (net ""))
 (segment (start 124 101) (end 124.5 101) (width 0.25) (layer "F.Cu") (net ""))
 (segment (start 150 101) (end 150.5 101) (width 0.25) (layer "F.Cu") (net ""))
 (segment (start 164 101) (end 164.5 101) (width 0.25) (layer "F.Cu") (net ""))
 (segment (start 159 101) (end 159.5 101) (width 0.25) (layer "F.Cu") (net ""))
 (segment (start 103 101) (end 103.5 101) (width 0.25) (layer "F.Cu") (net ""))
 (segment (start 180 101) (end 180.5 101) (width 0.25) (layer "F.Cu") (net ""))
 (segment (start 107 101) (end 107.5 101) (width 0.25) (layer "F.Cu") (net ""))
 (segment (start 123 101) (end 123.5 101) (width 0.25) (layer "F.Cu") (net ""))
 (segment (start 137 101) (end 137.5 101) (width 0.25) (layer "F.Cu") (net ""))
 (segment (start 101 101.5) (end 101.5 101.5) (width 0.25) (layer "F.Cu") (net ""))
 (segment (start 114 101) (end 114.5 101) (width 0.25) (layer "F.Cu") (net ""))
 (segment (start 171 101) (end 171.5 101) (width 0.25) (layer "F.Cu") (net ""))
 (segment (start 116 101.5) (end 116.5 101.5) (width 0.25) (layer "F.Cu") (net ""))
 (segment (start 126 101) (end 126.5 101) (width 0.25) (layer "F.Cu") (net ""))
 (segment (start 172 101) (end 172.5 101) (width 0.25) (layer "F.Cu") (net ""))
 (segment (start 104 101.5) (end 104.5 101.5) (width 0.25) (layer "F.Cu") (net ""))
 (segment (start 118 101.5) (end 118.5 101.5) (width 0.25) (layer "F.Cu") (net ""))
 (segment (start 107 101.5) (end 107.5 101.5) (width 0.25) (layer "F.Cu") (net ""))
 (segment (start 143 101) (end 143.5 101) (width 0.25) (layer "F.Cu") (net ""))
 (segment (start 118 101) (end 118.5 101) (width 0.25) (layer "F.Cu") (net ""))
 (segment (start 165 101) (end 165.5 101) (width 0.25) (layer "F.Cu") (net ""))
 (segment (start 103 101.5) (end 103.5 101.5) (width 0.25) (layer "F.Cu") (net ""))
 (segment (start 113 101.5) (end 113.5 101.5) (width 0.25) (layer "F.Cu") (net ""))
 (segment (start 102 101) (end 102.5 101) (width 0.25) (layer "F.Cu") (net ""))
 (segment (start 154 101) (end 154.5 101) (width 0.25) (layer "F.Cu") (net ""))
 (segment (start 161 101) (end 161.5 101) (width 0.25) (layer "F.Cu") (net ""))
 (segment (start 105 101.5) (end 105.5 101.5) (width 0.25) (layer "F.Cu") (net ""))
 (segment (start 138 101) (end 138.5 101) (width 0.25) (layer "F.Cu") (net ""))
 (segment (start 116 101) (end 116.5 101) (width 0.25) (layer "F.Cu") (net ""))
 (segment (start 133 101) (end 133.5 101) (width 0.25) (layer "F.Cu") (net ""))
 (segment (start 156 101) (end 156.5 101) (width 0.25) (layer "F.Cu") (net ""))
 (segment (start 109 101) (end 109.5 101) (width 0.25) (layer "F.Cu") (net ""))
 (segment (start 108 101.5) (end 108.5 101.5) (width 0.25) (layer "F.Cu") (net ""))
 (segment (start 158 101) (end 158.5 101) (width 0.25) (layer "F.Cu") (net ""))
 (segment (start 142 101) (end 142.5 101) (width 0.25) (layer "F.Cu") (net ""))
 (segment (start 120 101.5) (end 120.5 101.5) (width 0.25) (layer "F.Cu") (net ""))
 (segment (start 134 101) (end 134.5 101) (width 0.25) (layer "F.Cu") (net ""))
 (segment (start 132 101) (end 132.5 101) (width 0.25) (layer "F.Cu") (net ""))
 (segment (start 112 101.5) (end 112.5 101.5) (width 0.25) (layer "F.Cu") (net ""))
 (segment (start 108 101) (end 108.5 101) (width 0.25) (layer "F.Cu") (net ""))
 (segment (start 162 101) (end 162.5 101) (width 0.25) (layer "F.Cu") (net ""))
 (segment (start 130 101) (end 130.5 101) (width 0.25) (layer "F.Cu") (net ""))
 (segment (start 160 101) (end 160.5 101) (width 0.25) (layer "F.Cu") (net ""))
 (segment (start 119 101) (end 119.5 101) (width 0.25) (layer "F.Cu") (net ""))
 (segment (start 169 101) (end 169.5 101) (width 0.25) (layer "F.Cu") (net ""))
 (segment (start 120 101) (end 120.5 101) (width 0.25) (layer "F.Cu") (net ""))
 (segment (start 178 101) (end 178.5 101) (width 0.25) (layer "F.Cu") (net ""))
 (segment (start 166 101) (end 166.5 101) (width 0.25) (layer "F.Cu") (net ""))
 (segment (start 125 101) (end 125.5 101) (width 0.25) (layer "F.Cu") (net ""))
 (segment (start 129 101) (end 129.5 101) (width 0.25) (layer "F.Cu") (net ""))
 (segment (start 111 101.5) (end 111.5 101.5) (width 0.25) (layer "F.Cu") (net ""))
 (segment (start 145 101) (end 145.5 101) (width 0.25) (layer "F.Cu") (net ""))
 (segment (start 121 101) (end 121.5 101) (width 0.25) (layer "F.Cu") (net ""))
 (segment (start 117 101.5) (end 117.5 101.5) (width 0.25) (layer "F.Cu") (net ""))
 (segment (start 115 101.5) (end 115.5 101.5) (width 0.25) (layer "F.Cu") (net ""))
 (segment (start 111 101) (end 111.5 101) (width 0.25) (layer "F.Cu") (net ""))
 (segment (start 147 101) (end 147.5 101) (width 0.25) (layer "F.Cu") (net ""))
 (segment (start 139 101) (end 139.5 101) (width 0.25) (layer "F.Cu") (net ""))
 (segment (start 167 101) (end 167.5 101) (width 0.25) (layer "F.Cu") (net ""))
 (segment (start 106 101.5) (end 106.5 101.5) (width 0.25) (layer "F.Cu") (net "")))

